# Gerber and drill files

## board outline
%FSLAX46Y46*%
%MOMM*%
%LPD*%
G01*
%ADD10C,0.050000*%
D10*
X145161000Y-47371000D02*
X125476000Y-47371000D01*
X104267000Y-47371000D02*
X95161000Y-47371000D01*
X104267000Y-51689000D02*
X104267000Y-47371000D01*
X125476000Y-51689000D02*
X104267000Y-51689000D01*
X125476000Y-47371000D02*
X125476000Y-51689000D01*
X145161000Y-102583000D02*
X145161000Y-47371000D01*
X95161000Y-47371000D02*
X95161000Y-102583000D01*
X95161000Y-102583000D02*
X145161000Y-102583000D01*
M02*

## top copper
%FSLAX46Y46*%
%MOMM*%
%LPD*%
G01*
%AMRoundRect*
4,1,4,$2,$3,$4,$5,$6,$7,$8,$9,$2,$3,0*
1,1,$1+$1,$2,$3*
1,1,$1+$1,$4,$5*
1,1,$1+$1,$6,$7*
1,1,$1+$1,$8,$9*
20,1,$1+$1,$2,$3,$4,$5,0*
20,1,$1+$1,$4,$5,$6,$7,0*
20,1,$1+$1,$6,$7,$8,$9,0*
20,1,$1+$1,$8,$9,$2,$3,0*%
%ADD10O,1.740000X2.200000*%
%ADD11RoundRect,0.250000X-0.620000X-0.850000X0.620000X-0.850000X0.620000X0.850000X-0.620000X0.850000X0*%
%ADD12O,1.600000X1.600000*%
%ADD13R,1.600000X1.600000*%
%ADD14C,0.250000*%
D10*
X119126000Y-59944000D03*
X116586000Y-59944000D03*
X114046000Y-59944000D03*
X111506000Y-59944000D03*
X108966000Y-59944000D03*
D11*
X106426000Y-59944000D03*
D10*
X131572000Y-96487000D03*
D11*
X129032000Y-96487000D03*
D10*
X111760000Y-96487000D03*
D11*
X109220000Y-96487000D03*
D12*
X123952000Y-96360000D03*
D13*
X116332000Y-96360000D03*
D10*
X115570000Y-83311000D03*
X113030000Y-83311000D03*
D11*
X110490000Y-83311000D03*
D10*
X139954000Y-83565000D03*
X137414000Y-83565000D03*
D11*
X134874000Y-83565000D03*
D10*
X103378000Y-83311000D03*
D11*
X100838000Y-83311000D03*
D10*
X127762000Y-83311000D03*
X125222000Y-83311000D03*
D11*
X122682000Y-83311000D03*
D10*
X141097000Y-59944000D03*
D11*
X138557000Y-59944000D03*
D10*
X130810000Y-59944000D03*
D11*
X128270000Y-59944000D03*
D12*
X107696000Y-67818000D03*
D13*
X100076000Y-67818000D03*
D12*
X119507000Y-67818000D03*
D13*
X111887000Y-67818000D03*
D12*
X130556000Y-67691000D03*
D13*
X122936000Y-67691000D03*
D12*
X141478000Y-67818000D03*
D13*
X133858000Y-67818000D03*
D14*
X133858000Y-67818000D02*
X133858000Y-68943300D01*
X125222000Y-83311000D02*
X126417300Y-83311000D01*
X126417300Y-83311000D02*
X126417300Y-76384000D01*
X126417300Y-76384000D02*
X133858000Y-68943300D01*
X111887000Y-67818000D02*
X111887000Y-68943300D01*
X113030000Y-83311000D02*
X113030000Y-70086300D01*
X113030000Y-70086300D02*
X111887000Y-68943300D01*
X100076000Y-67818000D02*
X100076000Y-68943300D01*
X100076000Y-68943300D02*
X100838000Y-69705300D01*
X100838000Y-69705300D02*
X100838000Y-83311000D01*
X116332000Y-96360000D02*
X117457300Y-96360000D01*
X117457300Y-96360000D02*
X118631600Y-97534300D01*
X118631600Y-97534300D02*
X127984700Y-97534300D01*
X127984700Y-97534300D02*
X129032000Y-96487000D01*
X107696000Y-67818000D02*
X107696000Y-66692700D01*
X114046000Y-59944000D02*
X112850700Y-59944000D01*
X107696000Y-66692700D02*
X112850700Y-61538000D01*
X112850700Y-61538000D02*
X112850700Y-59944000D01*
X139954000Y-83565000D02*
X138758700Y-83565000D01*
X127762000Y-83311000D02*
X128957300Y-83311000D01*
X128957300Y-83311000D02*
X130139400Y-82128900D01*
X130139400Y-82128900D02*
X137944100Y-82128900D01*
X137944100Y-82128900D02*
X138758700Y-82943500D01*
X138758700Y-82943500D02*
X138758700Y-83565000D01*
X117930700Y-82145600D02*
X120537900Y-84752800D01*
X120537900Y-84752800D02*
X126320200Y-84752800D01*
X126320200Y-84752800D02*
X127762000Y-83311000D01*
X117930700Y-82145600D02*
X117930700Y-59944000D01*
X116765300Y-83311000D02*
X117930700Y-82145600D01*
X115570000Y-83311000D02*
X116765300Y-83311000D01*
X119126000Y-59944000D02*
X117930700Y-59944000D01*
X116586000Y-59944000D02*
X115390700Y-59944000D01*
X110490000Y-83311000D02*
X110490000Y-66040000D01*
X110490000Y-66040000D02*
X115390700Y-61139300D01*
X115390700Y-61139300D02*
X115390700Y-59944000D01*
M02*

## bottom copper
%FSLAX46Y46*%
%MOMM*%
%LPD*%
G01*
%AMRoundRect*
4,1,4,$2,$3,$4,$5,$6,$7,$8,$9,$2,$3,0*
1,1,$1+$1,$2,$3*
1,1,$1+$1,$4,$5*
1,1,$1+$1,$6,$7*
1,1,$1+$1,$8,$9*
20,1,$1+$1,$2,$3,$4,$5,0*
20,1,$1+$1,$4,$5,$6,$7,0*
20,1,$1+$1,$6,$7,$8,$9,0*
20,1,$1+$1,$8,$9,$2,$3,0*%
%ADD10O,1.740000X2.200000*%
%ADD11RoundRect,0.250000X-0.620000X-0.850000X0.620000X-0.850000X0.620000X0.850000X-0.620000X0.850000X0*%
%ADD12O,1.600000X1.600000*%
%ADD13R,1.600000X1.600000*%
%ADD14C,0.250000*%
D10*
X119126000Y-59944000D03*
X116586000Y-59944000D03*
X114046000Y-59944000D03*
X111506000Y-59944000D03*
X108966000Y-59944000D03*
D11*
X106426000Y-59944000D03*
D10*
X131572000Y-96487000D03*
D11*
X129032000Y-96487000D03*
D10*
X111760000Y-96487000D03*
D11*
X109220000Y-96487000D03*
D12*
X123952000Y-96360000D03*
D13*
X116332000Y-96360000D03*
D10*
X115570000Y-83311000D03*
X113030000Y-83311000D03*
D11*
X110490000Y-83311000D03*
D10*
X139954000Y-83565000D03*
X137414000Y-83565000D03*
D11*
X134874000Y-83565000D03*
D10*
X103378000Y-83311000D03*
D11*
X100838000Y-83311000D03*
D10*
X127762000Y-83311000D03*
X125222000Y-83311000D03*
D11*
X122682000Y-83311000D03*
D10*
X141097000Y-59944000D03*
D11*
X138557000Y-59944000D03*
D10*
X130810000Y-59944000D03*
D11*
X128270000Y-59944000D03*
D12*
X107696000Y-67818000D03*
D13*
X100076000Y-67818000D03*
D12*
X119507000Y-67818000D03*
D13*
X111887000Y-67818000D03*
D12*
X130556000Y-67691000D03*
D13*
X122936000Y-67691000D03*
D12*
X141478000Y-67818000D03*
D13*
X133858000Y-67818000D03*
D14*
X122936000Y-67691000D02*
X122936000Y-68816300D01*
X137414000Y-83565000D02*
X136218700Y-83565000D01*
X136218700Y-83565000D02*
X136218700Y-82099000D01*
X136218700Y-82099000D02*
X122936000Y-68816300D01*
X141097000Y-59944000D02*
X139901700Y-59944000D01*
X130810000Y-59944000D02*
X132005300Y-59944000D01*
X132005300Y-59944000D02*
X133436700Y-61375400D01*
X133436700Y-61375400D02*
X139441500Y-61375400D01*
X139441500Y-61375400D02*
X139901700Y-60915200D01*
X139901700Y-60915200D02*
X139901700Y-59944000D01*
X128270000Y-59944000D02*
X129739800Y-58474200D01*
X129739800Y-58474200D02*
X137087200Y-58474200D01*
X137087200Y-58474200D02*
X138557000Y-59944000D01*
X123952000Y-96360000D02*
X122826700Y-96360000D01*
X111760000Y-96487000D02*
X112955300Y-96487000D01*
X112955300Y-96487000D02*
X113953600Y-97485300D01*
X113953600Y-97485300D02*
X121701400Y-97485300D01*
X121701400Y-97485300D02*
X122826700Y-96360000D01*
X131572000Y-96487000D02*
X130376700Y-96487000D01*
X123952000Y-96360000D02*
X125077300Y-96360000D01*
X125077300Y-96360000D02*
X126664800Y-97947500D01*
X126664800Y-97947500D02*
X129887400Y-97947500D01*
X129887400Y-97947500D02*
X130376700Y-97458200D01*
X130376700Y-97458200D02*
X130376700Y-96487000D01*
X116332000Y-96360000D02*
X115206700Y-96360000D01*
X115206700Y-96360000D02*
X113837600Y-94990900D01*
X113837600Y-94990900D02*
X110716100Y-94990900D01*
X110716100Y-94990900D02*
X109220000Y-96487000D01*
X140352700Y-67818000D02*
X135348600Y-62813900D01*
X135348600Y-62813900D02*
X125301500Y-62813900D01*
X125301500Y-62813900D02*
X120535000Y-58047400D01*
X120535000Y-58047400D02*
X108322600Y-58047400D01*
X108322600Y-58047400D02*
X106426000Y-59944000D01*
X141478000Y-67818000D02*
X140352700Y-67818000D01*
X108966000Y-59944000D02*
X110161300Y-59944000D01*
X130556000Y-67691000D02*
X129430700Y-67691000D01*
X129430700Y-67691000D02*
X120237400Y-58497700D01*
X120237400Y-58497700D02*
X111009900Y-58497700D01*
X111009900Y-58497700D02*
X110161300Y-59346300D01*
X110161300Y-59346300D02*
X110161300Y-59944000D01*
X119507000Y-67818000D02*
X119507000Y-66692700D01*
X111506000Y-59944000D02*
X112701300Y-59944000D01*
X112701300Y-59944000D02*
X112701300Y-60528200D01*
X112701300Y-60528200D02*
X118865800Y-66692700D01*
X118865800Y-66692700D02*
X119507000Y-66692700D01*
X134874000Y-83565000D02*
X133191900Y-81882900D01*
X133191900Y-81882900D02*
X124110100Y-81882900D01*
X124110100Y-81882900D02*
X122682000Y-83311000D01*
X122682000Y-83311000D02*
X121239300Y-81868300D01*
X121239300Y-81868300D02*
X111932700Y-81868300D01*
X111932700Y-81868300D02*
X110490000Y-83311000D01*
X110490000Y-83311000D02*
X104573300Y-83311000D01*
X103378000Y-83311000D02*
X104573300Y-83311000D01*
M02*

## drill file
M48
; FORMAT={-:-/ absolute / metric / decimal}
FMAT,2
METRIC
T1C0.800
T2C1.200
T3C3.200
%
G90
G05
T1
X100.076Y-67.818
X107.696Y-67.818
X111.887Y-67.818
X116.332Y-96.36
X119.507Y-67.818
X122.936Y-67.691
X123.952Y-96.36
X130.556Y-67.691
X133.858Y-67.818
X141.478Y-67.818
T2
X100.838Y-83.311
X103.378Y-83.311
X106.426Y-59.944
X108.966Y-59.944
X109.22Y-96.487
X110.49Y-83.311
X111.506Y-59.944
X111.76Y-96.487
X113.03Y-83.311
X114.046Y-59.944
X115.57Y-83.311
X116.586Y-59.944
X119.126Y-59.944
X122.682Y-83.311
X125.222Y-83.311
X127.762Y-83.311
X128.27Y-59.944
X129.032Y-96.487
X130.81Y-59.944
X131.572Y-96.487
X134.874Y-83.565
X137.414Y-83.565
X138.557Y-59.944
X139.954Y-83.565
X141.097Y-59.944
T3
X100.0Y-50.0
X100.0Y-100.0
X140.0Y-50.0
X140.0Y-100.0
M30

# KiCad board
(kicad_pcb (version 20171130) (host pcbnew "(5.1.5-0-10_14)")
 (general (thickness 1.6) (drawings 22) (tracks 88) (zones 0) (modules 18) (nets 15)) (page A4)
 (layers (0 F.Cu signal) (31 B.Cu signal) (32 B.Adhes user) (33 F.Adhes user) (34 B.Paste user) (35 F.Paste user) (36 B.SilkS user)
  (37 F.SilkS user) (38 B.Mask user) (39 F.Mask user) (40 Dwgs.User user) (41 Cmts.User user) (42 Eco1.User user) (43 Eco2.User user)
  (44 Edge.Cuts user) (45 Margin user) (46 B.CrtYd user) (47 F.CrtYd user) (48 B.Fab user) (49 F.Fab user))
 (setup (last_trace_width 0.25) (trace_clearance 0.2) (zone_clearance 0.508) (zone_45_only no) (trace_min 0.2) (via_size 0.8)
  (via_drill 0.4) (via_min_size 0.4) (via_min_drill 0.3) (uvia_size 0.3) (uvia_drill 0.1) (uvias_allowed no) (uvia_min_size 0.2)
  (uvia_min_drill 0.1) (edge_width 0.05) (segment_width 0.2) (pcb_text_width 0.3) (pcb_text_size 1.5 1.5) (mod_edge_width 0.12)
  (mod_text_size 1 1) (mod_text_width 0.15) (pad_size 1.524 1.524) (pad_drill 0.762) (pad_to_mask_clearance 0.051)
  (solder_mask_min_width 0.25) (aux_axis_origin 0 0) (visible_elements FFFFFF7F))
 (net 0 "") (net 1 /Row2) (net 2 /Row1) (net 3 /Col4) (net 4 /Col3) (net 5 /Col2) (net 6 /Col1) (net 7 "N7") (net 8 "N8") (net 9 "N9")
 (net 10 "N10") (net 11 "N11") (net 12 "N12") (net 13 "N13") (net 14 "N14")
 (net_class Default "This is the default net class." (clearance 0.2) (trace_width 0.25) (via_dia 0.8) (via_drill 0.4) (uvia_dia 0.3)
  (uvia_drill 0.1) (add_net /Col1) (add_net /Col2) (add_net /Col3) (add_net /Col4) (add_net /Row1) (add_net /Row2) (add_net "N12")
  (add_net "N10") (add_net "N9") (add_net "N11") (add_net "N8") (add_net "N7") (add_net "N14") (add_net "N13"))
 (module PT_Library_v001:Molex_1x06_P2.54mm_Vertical (layer F.Cu) (at 106.426 59.944)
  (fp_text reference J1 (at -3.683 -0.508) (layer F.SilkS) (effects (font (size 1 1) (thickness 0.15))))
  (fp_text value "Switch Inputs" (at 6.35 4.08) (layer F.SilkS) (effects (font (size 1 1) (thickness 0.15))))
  (pad 6 thru_hole oval (at 12.7 0) (size 1.74 2.2) (drill 1.2) (layers *.Cu *.Mask) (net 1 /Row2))
  (pad 5 thru_hole oval (at 10.16 0) (size 1.74 2.2) (drill 1.2) (layers *.Cu *.Mask) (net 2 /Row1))
  (pad 4 thru_hole oval (at 7.62 0) (size 1.74 2.2) (drill 1.2) (layers *.Cu *.Mask) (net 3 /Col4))
  (pad 3 thru_hole oval (at 5.08 0) (size 1.74 2.2) (drill 1.2) (layers *.Cu *.Mask) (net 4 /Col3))
  (pad 2 thru_hole oval (at 2.54 0) (size 1.74 2.2) (drill 1.2) (layers *.Cu *.Mask) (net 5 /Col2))
  (pad 1 thru_hole roundrect (at 0 0) (size 1.74 2.2) (drill 1.2) (layers *.Cu *.Mask) (roundrect_rratio 0.143678) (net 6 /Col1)))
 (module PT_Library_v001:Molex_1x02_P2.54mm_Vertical (layer F.Cu) (at 129.032 96.487)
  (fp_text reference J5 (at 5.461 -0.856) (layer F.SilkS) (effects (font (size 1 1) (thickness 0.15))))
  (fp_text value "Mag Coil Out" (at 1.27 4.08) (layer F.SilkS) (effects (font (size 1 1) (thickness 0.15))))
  (pad 2 thru_hole oval (at 2.54 0) (size 1.74 2.2) (drill 1.2) (layers *.Cu *.Mask) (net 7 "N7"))
  (pad 1 thru_hole roundrect (at 0 0) (size 1.74 2.2) (drill 1.2) (layers *.Cu *.Mask) (roundrect_rratio 0.143678) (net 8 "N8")))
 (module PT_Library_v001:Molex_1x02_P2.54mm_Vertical (layer F.Cu) (at 109.22 96.487)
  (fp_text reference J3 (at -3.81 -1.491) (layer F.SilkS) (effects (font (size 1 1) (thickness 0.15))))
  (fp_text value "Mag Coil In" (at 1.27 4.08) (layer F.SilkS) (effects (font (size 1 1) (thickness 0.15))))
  (pad 2 thru_hole oval (at 2.54 0) (size 1.74 2.2) (drill 1.2) (layers *.Cu *.Mask) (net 7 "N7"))
  (pad 1 thru_hole roundrect (at 0 0) (size 1.74 2.2) (drill 1.2) (layers *.Cu *.Mask) (roundrect_rratio 0.143678) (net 8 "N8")))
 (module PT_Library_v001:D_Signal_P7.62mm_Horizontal (layer F.Cu) (at 116.332 96.36)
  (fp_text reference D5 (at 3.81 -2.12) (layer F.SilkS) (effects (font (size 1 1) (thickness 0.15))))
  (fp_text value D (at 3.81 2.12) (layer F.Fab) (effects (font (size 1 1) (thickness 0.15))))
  (pad 2 thru_hole oval (at 7.62 0) (size 1.6 1.6) (drill 0.8) (layers *.Cu *.Mask) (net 7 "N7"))
  (pad 1 thru_hole rect (at 0 0) (size 1.6 1.6) (drill 0.8) (layers *.Cu *.Mask) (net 8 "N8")))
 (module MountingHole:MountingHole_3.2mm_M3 (layer F.Cu) (at 140 100)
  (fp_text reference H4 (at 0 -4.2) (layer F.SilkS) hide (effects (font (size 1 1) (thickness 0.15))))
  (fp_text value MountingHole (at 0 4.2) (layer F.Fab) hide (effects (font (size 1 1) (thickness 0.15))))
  (pad 1 np_thru_hole circle (at 0 0) (size 3.2 3.2) (drill 3.2) (layers *.Cu *.Mask)))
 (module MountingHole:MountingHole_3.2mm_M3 (layer F.Cu) (at 100 100)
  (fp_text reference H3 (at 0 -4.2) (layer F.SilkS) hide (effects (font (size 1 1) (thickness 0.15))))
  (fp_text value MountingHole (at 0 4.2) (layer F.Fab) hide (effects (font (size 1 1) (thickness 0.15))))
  (pad 1 np_thru_hole circle (at 0 0) (size 3.2 3.2) (drill 3.2) (layers *.Cu *.Mask)))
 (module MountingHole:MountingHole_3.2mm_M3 (layer F.Cu) (at 140 50)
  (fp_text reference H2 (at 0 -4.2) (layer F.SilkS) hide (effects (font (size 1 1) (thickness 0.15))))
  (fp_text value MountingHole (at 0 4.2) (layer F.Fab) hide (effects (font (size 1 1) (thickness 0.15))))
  (pad 1 np_thru_hole circle (at 0 0) (size 3.2 3.2) (drill 3.2) (layers *.Cu *.Mask)))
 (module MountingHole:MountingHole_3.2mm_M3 (layer F.Cu) (at 100 50)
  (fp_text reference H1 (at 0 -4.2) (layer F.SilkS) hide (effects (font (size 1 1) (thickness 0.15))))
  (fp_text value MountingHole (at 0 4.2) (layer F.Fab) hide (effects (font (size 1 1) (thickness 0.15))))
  (pad 1 np_thru_hole circle (at 0 0) (size 3.2 3.2) (drill 3.2) (layers *.Cu *.Mask)))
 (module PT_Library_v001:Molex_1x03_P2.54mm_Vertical (layer F.Cu) (at 110.49 83.311)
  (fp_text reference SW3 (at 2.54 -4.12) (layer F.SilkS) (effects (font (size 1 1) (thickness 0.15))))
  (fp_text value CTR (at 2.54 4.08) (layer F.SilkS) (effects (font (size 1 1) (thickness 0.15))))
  (pad 3 thru_hole oval (at 5.08 0) (size 1.74 2.2) (drill 1.2) (layers *.Cu *.Mask) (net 1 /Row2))
  (pad 2 thru_hole oval (at 2.54 0) (size 1.74 2.2) (drill 1.2) (layers *.Cu *.Mask) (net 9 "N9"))
  (pad 1 thru_hole roundrect (at 0 0) (size 1.74 2.2) (drill 1.2) (layers *.Cu *.Mask) (roundrect_rratio 0.143678) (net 2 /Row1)))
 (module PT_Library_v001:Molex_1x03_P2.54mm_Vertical (layer F.Cu) (at 134.874 83.565)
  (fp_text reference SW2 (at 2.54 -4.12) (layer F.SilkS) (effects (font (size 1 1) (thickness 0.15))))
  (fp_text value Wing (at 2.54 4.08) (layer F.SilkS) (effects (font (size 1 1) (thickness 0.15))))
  (pad 3 thru_hole oval (at 5.08 0) (size 1.74 2.2) (drill 1.2) (layers *.Cu *.Mask) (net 1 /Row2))
  (pad 2 thru_hole oval (at 2.54 0) (size 1.74 2.2) (drill 1.2) (layers *.Cu *.Mask) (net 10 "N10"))
  (pad 1 thru_hole roundrect (at 0 0) (size 1.74 2.2) (drill 1.2) (layers *.Cu *.Mask) (roundrect_rratio 0.143678) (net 2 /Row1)))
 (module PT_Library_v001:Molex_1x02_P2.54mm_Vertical (layer F.Cu) (at 100.838 83.311)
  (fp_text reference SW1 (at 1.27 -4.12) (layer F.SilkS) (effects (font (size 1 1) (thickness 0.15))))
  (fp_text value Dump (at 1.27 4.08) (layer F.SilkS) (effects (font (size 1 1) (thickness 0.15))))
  (pad 2 thru_hole oval (at 2.54 0) (size 1.74 2.2) (drill 1.2) (layers *.Cu *.Mask) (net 2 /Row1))
  (pad 1 thru_hole roundrect (at 0 0) (size 1.74 2.2) (drill 1.2) (layers *.Cu *.Mask) (roundrect_rratio 0.143678) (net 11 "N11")))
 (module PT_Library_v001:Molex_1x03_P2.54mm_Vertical (layer F.Cu) (at 122.682 83.311)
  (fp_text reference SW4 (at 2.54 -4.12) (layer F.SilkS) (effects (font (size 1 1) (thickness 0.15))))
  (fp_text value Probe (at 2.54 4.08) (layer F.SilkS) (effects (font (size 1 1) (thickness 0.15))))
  (pad 3 thru_hole oval (at 5.08 0) (size 1.74 2.2) (drill 1.2) (layers *.Cu *.Mask) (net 1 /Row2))
  (pad 2 thru_hole oval (at 2.54 0) (size 1.74 2.2) (drill 1.2) (layers *.Cu *.Mask) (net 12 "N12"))
  (pad 1 thru_hole roundrect (at 0 0) (size 1.74 2.2) (drill 1.2) (layers *.Cu *.Mask) (roundrect_rratio 0.143678) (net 2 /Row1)))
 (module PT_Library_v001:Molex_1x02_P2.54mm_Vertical (layer F.Cu) (at 138.557 59.944)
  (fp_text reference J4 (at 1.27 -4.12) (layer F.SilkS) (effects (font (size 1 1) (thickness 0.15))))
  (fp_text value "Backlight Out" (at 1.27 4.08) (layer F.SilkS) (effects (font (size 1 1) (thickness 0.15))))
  (pad 2 thru_hole oval (at 2.54 0) (size 1.74 2.2) (drill 1.2) (layers *.Cu *.Mask) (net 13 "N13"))
  (pad 1 thru_hole roundrect (at 0 0) (size 1.74 2.2) (drill 1.2) (layers *.Cu *.Mask) (roundrect_rratio 0.143678) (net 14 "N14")))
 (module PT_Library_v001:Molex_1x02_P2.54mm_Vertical (layer F.Cu) (at 128.27 59.944)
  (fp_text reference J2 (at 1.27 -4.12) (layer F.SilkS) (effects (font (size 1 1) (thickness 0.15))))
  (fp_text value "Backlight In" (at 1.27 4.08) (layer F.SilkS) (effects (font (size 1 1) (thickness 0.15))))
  (pad 2 thru_hole oval (at 2.54 0) (size 1.74 2.2) (drill 1.2) (layers *.Cu *.Mask) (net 13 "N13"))
  (pad 1 thru_hole roundrect (at 0 0) (size 1.74 2.2) (drill 1.2) (layers *.Cu *.Mask) (roundrect_rratio 0.143678) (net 14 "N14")))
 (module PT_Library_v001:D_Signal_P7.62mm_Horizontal (layer F.Cu) (at 100.076 67.818)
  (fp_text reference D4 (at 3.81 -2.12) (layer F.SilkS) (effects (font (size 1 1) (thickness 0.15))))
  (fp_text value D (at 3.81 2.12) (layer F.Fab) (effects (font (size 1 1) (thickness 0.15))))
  (pad 2 thru_hole oval (at 7.62 0) (size 1.6 1.6) (drill 0.8) (layers *.Cu *.Mask) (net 3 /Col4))
  (pad 1 thru_hole rect (at 0 0) (size 1.6 1.6) (drill 0.8) (layers *.Cu *.Mask) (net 11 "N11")))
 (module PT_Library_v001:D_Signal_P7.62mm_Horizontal (layer F.Cu) (at 111.887 67.818)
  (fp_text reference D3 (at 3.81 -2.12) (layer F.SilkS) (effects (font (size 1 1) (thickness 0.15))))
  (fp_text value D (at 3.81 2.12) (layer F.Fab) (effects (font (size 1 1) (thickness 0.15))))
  (pad 2 thru_hole oval (at 7.62 0) (size 1.6 1.6) (drill 0.8) (layers *.Cu *.Mask) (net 4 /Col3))
  (pad 1 thru_hole rect (at 0 0) (size 1.6 1.6) (drill 0.8) (layers *.Cu *.Mask) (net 9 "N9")))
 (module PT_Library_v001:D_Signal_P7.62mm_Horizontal (layer F.Cu) (at 122.936 67.691)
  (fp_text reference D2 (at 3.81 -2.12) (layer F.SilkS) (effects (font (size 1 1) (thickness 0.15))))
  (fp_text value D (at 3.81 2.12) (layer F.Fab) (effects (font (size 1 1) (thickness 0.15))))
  (pad 2 thru_hole oval (at 7.62 0) (size 1.6 1.6) (drill 0.8) (layers *.Cu *.Mask) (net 5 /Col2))
  (pad 1 thru_hole rect (at 0 0) (size 1.6 1.6) (drill 0.8) (layers *.Cu *.Mask) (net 10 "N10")))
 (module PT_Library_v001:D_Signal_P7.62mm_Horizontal (layer F.Cu) (at 133.858 67.818)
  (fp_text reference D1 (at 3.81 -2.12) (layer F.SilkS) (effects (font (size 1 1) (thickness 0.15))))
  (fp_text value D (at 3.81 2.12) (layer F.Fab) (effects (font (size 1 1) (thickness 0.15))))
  (pad 2 thru_hole oval (at 7.62 0) (size 1.6 1.6) (drill 0.8) (layers *.Cu *.Mask) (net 6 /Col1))
  (pad 1 thru_hole rect (at 0 0) (size 1.6 1.6) (drill 0.8) (layers *.Cu *.Mask) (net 12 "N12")))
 (gr_line (start 145.161 47.371) (end 125.476 47.371) (layer Edge.Cuts) (width 0.05))
 (gr_line (start 104.267 47.371) (end 95.161 47.371) (layer Edge.Cuts) (width 0.05))
 (gr_line (start 104.267 51.689) (end 104.267 47.371) (layer Edge.Cuts) (width 0.05))
 (gr_line (start 125.476 51.689) (end 104.267 51.689) (layer Edge.Cuts) (width 0.05))
 (gr_line (start 125.476 47.371) (end 125.476 51.689) (layer Edge.Cuts) (width 0.05))
 (gr_line (start 145.161 102.583) (end 145.161 47.371) (layer Edge.Cuts) (width 0.05))
 (gr_line (start 95.161 47.371) (end 95.161 102.583) (layer Edge.Cuts) (width 0.05))
 (gr_line (start 95.161 102.583) (end 145.161 102.583) (layer Edge.Cuts) (width 0.05))
 (segment (start 133.858 67.818) (end 133.858 68.9433) (width 0.25) (layer F.Cu) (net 12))
 (segment (start 125.222 83.311) (end 126.4173 83.311) (width 0.25) (layer F.Cu) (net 12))
 (segment (start 126.4173 83.311) (end 126.4173 76.384) (width 0.25) (layer F.Cu) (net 12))
 (segment (start 126.4173 76.384) (end 133.858 68.9433) (width 0.25) (layer F.Cu) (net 12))
 (segment (start 122.936 67.691) (end 122.936 68.8163) (width 0.25) (layer B.Cu) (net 10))
 (segment (start 137.414 83.565) (end 136.2187 83.565) (width 0.25) (layer B.Cu) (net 10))
 (segment (start 136.2187 83.565) (end 136.2187 82.099) (width 0.25) (layer B.Cu) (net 10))
 (segment (start 136.2187 82.099) (end 122.936 68.8163) (width 0.25) (layer B.Cu) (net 10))
 (segment (start 111.887 67.818) (end 111.887 68.9433) (width 0.25) (layer F.Cu) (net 9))
 (segment (start 113.03 83.311) (end 113.03 70.0863) (width 0.25) (layer F.Cu) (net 9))
 (segment (start 113.03 70.0863) (end 111.887 68.9433) (width 0.25) (layer F.Cu) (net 9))
 (segment (start 100.076 67.818) (end 100.076 68.9433) (width 0.25) (layer F.Cu) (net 11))
 (segment (start 100.076 68.9433) (end 100.838 69.7053) (width 0.25) (layer F.Cu) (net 11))
 (segment (start 100.838 69.7053) (end 100.838 83.311) (width 0.25) (layer F.Cu) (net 11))
 (segment (start 141.097 59.944) (end 139.9017 59.944) (width 0.25) (layer B.Cu) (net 13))
 (segment (start 130.81 59.944) (end 132.0053 59.944) (width 0.25) (layer B.Cu) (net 13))
 (segment (start 132.0053 59.944) (end 133.4367 61.3754) (width 0.25) (layer B.Cu) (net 13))
 (segment (start 133.4367 61.3754) (end 139.4415 61.3754) (width 0.25) (layer B.Cu) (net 13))
 (segment (start 139.4415 61.3754) (end 139.9017 60.9152) (width 0.25) (layer B.Cu) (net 13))
 (segment (start 139.9017 60.9152) (end 139.9017 59.944) (width 0.25) (layer B.Cu) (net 13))
 (segment (start 128.27 59.944) (end 129.7398 58.4742) (width 0.25) (layer B.Cu) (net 14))
 (segment (start 129.7398 58.4742) (end 137.0872 58.4742) (width 0.25) (layer B.Cu) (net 14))
 (segment (start 137.0872 58.4742) (end 138.557 59.944) (width 0.25) (layer B.Cu) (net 14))
 (segment (start 123.952 96.36) (end 122.8267 96.36) (width 0.25) (layer B.Cu) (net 7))
 (segment (start 111.76 96.487) (end 112.9553 96.487) (width 0.25) (layer B.Cu) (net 7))
 (segment (start 112.9553 96.487) (end 113.9536 97.4853) (width 0.25) (layer B.Cu) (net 7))
 (segment (start 113.9536 97.4853) (end 121.7014 97.4853) (width 0.25) (layer B.Cu) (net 7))
 (segment (start 121.7014 97.4853) (end 122.8267 96.36) (width 0.25) (layer B.Cu) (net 7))
 (segment (start 131.572 96.487) (end 130.3767 96.487) (width 0.25) (layer B.Cu) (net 7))
 (segment (start 123.952 96.36) (end 125.0773 96.36) (width 0.25) (layer B.Cu) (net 7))
 (segment (start 125.0773 96.36) (end 126.6648 97.9475) (width 0.25) (layer B.Cu) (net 7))
 (segment (start 126.6648 97.9475) (end 129.8874 97.9475) (width 0.25) (layer B.Cu) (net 7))
 (segment (start 129.8874 97.9475) (end 130.3767 97.4582) (width 0.25) (layer B.Cu) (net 7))
 (segment (start 130.3767 97.4582) (end 130.3767 96.487) (width 0.25) (layer B.Cu) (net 7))
 (segment (start 116.332 96.36) (end 117.4573 96.36) (width 0.25) (layer F.Cu) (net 8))
 (segment (start 117.4573 96.36) (end 118.6316 97.5343) (width 0.25) (layer F.Cu) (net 8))
 (segment (start 118.6316 97.5343) (end 127.9847 97.5343) (width 0.25) (layer F.Cu) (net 8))
 (segment (start 127.9847 97.5343) (end 129.032 96.487) (width 0.25) (layer F.Cu) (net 8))
 (segment (start 116.332 96.36) (end 115.2067 96.36) (width 0.25) (layer B.Cu) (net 8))
 (segment (start 115.2067 96.36) (end 113.8376 94.9909) (width 0.25) (layer B.Cu) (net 8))
 (segment (start 113.8376 94.9909) (end 110.7161 94.9909) (width 0.25) (layer B.Cu) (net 8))
 (segment (start 110.7161 94.9909) (end 109.22 96.487) (width 0.25) (layer B.Cu) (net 8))
 (segment (start 140.3527 67.818) (end 135.3486 62.8139) (width 0.25) (layer B.Cu) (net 6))
 (segment (start 135.3486 62.8139) (end 125.3015 62.8139) (width 0.25) (layer B.Cu) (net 6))
 (segment (start 125.3015 62.8139) (end 120.535 58.0474) (width 0.25) (layer B.Cu) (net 6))
 (segment (start 120.535 58.0474) (end 108.3226 58.0474) (width 0.25) (layer B.Cu) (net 6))
 (segment (start 108.3226 58.0474) (end 106.426 59.944) (width 0.25) (layer B.Cu) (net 6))
 (segment (start 141.478 67.818) (end 140.3527 67.818) (width 0.25) (layer B.Cu) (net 6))
 (segment (start 108.966 59.944) (end 110.1613 59.944) (width 0.25) (layer B.Cu) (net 5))
 (segment (start 130.556 67.691) (end 129.4307 67.691) (width 0.25) (layer B.Cu) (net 5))
 (segment (start 129.4307 67.691) (end 120.2374 58.4977) (width 0.25) (layer B.Cu) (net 5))
 (segment (start 120.2374 58.4977) (end 111.0099 58.4977) (width 0.25) (layer B.Cu) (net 5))
 (segment (start 111.0099 58.4977) (end 110.1613 59.3463) (width 0.25) (layer B.Cu) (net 5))
 (segment (start 110.1613 59.3463) (end 110.1613 59.944) (width 0.25) (layer B.Cu) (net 5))
 (segment (start 119.507 67.818) (end 119.507 66.6927) (width 0.25) (layer B.Cu) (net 4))
 (segment (start 111.506 59.944) (end 112.7013 59.944) (width 0.25) (layer B.Cu) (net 4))
 (segment (start 112.7013 59.944) (end 112.7013 60.5282) (width 0.25) (layer B.Cu) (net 4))
 (segment (start 112.7013 60.5282) (end 118.8658 66.6927) (width 0.25) (layer B.Cu) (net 4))
 (segment (start 118.8658 66.6927) (end 119.507 66.6927) (width 0.25) (layer B.Cu) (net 4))
 (segment (start 107.696 67.818) (end 107.696 66.6927) (width 0.25) (layer F.Cu) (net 3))
 (segment (start 114.046 59.944) (end 112.8507 59.944) (width 0.25) (layer F.Cu) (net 3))
 (segment (start 107.696 66.6927) (end 112.8507 61.538) (width 0.25) (layer F.Cu) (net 3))
 (segment (start 112.8507 61.538) (end 112.8507 59.944) (width 0.25) (layer F.Cu) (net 3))
 (segment (start 139.954 83.565) (end 138.7587 83.565) (width 0.25) (layer F.Cu) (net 1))
 (segment (start 127.762 83.311) (end 128.9573 83.311) (width 0.25) (layer F.Cu) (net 1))
 (segment (start 128.9573 83.311) (end 130.1394 82.1289) (width 0.25) (layer F.Cu) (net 1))
 (segment (start 130.1394 82.1289) (end 137.9441 82.1289) (width 0.25) (layer F.Cu) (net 1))
 (segment (start 137.9441 82.1289) (end 138.7587 82.9435) (width 0.25) (layer F.Cu) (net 1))
 (segment (start 138.7587 82.9435) (end 138.7587 83.565) (width 0.25) (layer F.Cu) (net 1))
 (segment (start 117.9307 82.1456) (end 120.5379 84.7528) (width 0.25) (layer F.Cu) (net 1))
 (segment (start 120.5379 84.7528) (end 126.3202 84.7528) (width 0.25) (layer F.Cu) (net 1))
 (segment (start 126.3202 84.7528) (end 127.762 83.311) (width 0.25) (layer F.Cu) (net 1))
 (segment (start 117.9307 82.1456) (end 117.9307 59.944) (width 0.25) (layer F.Cu) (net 1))
 (segment (start 116.7653 83.311) (end 117.9307 82.1456) (width 0.25) (layer F.Cu) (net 1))
 (segment (start 115.57 83.311) (end 116.7653 83.311) (width 0.25) (layer F.Cu) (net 1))
 (segment (start 119.126 59.944) (end 117.9307 59.944) (width 0.25) (layer F.Cu) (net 1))
 (segment (start 116.586 59.944) (end 115.3907 59.944) (width 0.25) (layer F.Cu) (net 2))
 (segment (start 110.49 83.311) (end 110.49 66.04) (width 0.25) (layer F.Cu) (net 2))
 (segment (start 110.49 66.04) (end 115.3907 61.1393) (width 0.25) (layer F.Cu) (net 2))
 (segment (start 115.3907 61.1393) (end 115.3907 59.944) (width 0.25) (layer F.Cu) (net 2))
 (segment (start 134.874 83.565) (end 133.1919 81.8829) (width 0.25) (layer B.Cu) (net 2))
 (segment (start 133.1919 81.8829) (end 124.1101 81.8829) (width 0.25) (layer B.Cu) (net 2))
 (segment (start 124.1101 81.8829) (end 122.682 83.311) (width 0.25) (layer B.Cu) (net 2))
 (segment (start 122.682 83.311) (end 121.2393 81.8683) (width 0.25) (layer B.Cu) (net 2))
 (segment (start 121.2393 81.8683) (end 111.9327 81.8683) (width 0.25) (layer B.Cu) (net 2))
 (segment (start 111.9327 81.8683) (end 110.49 83.311) (width 0.25) (layer B.Cu) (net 2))
 (segment (start 110.49 83.311) (end 104.5733 83.311) (width 0.25) (layer B.Cu) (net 2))
 (segment (start 103.378 83.311) (end 104.5733 83.311) (width 0.25) (layer B.Cu) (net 2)))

